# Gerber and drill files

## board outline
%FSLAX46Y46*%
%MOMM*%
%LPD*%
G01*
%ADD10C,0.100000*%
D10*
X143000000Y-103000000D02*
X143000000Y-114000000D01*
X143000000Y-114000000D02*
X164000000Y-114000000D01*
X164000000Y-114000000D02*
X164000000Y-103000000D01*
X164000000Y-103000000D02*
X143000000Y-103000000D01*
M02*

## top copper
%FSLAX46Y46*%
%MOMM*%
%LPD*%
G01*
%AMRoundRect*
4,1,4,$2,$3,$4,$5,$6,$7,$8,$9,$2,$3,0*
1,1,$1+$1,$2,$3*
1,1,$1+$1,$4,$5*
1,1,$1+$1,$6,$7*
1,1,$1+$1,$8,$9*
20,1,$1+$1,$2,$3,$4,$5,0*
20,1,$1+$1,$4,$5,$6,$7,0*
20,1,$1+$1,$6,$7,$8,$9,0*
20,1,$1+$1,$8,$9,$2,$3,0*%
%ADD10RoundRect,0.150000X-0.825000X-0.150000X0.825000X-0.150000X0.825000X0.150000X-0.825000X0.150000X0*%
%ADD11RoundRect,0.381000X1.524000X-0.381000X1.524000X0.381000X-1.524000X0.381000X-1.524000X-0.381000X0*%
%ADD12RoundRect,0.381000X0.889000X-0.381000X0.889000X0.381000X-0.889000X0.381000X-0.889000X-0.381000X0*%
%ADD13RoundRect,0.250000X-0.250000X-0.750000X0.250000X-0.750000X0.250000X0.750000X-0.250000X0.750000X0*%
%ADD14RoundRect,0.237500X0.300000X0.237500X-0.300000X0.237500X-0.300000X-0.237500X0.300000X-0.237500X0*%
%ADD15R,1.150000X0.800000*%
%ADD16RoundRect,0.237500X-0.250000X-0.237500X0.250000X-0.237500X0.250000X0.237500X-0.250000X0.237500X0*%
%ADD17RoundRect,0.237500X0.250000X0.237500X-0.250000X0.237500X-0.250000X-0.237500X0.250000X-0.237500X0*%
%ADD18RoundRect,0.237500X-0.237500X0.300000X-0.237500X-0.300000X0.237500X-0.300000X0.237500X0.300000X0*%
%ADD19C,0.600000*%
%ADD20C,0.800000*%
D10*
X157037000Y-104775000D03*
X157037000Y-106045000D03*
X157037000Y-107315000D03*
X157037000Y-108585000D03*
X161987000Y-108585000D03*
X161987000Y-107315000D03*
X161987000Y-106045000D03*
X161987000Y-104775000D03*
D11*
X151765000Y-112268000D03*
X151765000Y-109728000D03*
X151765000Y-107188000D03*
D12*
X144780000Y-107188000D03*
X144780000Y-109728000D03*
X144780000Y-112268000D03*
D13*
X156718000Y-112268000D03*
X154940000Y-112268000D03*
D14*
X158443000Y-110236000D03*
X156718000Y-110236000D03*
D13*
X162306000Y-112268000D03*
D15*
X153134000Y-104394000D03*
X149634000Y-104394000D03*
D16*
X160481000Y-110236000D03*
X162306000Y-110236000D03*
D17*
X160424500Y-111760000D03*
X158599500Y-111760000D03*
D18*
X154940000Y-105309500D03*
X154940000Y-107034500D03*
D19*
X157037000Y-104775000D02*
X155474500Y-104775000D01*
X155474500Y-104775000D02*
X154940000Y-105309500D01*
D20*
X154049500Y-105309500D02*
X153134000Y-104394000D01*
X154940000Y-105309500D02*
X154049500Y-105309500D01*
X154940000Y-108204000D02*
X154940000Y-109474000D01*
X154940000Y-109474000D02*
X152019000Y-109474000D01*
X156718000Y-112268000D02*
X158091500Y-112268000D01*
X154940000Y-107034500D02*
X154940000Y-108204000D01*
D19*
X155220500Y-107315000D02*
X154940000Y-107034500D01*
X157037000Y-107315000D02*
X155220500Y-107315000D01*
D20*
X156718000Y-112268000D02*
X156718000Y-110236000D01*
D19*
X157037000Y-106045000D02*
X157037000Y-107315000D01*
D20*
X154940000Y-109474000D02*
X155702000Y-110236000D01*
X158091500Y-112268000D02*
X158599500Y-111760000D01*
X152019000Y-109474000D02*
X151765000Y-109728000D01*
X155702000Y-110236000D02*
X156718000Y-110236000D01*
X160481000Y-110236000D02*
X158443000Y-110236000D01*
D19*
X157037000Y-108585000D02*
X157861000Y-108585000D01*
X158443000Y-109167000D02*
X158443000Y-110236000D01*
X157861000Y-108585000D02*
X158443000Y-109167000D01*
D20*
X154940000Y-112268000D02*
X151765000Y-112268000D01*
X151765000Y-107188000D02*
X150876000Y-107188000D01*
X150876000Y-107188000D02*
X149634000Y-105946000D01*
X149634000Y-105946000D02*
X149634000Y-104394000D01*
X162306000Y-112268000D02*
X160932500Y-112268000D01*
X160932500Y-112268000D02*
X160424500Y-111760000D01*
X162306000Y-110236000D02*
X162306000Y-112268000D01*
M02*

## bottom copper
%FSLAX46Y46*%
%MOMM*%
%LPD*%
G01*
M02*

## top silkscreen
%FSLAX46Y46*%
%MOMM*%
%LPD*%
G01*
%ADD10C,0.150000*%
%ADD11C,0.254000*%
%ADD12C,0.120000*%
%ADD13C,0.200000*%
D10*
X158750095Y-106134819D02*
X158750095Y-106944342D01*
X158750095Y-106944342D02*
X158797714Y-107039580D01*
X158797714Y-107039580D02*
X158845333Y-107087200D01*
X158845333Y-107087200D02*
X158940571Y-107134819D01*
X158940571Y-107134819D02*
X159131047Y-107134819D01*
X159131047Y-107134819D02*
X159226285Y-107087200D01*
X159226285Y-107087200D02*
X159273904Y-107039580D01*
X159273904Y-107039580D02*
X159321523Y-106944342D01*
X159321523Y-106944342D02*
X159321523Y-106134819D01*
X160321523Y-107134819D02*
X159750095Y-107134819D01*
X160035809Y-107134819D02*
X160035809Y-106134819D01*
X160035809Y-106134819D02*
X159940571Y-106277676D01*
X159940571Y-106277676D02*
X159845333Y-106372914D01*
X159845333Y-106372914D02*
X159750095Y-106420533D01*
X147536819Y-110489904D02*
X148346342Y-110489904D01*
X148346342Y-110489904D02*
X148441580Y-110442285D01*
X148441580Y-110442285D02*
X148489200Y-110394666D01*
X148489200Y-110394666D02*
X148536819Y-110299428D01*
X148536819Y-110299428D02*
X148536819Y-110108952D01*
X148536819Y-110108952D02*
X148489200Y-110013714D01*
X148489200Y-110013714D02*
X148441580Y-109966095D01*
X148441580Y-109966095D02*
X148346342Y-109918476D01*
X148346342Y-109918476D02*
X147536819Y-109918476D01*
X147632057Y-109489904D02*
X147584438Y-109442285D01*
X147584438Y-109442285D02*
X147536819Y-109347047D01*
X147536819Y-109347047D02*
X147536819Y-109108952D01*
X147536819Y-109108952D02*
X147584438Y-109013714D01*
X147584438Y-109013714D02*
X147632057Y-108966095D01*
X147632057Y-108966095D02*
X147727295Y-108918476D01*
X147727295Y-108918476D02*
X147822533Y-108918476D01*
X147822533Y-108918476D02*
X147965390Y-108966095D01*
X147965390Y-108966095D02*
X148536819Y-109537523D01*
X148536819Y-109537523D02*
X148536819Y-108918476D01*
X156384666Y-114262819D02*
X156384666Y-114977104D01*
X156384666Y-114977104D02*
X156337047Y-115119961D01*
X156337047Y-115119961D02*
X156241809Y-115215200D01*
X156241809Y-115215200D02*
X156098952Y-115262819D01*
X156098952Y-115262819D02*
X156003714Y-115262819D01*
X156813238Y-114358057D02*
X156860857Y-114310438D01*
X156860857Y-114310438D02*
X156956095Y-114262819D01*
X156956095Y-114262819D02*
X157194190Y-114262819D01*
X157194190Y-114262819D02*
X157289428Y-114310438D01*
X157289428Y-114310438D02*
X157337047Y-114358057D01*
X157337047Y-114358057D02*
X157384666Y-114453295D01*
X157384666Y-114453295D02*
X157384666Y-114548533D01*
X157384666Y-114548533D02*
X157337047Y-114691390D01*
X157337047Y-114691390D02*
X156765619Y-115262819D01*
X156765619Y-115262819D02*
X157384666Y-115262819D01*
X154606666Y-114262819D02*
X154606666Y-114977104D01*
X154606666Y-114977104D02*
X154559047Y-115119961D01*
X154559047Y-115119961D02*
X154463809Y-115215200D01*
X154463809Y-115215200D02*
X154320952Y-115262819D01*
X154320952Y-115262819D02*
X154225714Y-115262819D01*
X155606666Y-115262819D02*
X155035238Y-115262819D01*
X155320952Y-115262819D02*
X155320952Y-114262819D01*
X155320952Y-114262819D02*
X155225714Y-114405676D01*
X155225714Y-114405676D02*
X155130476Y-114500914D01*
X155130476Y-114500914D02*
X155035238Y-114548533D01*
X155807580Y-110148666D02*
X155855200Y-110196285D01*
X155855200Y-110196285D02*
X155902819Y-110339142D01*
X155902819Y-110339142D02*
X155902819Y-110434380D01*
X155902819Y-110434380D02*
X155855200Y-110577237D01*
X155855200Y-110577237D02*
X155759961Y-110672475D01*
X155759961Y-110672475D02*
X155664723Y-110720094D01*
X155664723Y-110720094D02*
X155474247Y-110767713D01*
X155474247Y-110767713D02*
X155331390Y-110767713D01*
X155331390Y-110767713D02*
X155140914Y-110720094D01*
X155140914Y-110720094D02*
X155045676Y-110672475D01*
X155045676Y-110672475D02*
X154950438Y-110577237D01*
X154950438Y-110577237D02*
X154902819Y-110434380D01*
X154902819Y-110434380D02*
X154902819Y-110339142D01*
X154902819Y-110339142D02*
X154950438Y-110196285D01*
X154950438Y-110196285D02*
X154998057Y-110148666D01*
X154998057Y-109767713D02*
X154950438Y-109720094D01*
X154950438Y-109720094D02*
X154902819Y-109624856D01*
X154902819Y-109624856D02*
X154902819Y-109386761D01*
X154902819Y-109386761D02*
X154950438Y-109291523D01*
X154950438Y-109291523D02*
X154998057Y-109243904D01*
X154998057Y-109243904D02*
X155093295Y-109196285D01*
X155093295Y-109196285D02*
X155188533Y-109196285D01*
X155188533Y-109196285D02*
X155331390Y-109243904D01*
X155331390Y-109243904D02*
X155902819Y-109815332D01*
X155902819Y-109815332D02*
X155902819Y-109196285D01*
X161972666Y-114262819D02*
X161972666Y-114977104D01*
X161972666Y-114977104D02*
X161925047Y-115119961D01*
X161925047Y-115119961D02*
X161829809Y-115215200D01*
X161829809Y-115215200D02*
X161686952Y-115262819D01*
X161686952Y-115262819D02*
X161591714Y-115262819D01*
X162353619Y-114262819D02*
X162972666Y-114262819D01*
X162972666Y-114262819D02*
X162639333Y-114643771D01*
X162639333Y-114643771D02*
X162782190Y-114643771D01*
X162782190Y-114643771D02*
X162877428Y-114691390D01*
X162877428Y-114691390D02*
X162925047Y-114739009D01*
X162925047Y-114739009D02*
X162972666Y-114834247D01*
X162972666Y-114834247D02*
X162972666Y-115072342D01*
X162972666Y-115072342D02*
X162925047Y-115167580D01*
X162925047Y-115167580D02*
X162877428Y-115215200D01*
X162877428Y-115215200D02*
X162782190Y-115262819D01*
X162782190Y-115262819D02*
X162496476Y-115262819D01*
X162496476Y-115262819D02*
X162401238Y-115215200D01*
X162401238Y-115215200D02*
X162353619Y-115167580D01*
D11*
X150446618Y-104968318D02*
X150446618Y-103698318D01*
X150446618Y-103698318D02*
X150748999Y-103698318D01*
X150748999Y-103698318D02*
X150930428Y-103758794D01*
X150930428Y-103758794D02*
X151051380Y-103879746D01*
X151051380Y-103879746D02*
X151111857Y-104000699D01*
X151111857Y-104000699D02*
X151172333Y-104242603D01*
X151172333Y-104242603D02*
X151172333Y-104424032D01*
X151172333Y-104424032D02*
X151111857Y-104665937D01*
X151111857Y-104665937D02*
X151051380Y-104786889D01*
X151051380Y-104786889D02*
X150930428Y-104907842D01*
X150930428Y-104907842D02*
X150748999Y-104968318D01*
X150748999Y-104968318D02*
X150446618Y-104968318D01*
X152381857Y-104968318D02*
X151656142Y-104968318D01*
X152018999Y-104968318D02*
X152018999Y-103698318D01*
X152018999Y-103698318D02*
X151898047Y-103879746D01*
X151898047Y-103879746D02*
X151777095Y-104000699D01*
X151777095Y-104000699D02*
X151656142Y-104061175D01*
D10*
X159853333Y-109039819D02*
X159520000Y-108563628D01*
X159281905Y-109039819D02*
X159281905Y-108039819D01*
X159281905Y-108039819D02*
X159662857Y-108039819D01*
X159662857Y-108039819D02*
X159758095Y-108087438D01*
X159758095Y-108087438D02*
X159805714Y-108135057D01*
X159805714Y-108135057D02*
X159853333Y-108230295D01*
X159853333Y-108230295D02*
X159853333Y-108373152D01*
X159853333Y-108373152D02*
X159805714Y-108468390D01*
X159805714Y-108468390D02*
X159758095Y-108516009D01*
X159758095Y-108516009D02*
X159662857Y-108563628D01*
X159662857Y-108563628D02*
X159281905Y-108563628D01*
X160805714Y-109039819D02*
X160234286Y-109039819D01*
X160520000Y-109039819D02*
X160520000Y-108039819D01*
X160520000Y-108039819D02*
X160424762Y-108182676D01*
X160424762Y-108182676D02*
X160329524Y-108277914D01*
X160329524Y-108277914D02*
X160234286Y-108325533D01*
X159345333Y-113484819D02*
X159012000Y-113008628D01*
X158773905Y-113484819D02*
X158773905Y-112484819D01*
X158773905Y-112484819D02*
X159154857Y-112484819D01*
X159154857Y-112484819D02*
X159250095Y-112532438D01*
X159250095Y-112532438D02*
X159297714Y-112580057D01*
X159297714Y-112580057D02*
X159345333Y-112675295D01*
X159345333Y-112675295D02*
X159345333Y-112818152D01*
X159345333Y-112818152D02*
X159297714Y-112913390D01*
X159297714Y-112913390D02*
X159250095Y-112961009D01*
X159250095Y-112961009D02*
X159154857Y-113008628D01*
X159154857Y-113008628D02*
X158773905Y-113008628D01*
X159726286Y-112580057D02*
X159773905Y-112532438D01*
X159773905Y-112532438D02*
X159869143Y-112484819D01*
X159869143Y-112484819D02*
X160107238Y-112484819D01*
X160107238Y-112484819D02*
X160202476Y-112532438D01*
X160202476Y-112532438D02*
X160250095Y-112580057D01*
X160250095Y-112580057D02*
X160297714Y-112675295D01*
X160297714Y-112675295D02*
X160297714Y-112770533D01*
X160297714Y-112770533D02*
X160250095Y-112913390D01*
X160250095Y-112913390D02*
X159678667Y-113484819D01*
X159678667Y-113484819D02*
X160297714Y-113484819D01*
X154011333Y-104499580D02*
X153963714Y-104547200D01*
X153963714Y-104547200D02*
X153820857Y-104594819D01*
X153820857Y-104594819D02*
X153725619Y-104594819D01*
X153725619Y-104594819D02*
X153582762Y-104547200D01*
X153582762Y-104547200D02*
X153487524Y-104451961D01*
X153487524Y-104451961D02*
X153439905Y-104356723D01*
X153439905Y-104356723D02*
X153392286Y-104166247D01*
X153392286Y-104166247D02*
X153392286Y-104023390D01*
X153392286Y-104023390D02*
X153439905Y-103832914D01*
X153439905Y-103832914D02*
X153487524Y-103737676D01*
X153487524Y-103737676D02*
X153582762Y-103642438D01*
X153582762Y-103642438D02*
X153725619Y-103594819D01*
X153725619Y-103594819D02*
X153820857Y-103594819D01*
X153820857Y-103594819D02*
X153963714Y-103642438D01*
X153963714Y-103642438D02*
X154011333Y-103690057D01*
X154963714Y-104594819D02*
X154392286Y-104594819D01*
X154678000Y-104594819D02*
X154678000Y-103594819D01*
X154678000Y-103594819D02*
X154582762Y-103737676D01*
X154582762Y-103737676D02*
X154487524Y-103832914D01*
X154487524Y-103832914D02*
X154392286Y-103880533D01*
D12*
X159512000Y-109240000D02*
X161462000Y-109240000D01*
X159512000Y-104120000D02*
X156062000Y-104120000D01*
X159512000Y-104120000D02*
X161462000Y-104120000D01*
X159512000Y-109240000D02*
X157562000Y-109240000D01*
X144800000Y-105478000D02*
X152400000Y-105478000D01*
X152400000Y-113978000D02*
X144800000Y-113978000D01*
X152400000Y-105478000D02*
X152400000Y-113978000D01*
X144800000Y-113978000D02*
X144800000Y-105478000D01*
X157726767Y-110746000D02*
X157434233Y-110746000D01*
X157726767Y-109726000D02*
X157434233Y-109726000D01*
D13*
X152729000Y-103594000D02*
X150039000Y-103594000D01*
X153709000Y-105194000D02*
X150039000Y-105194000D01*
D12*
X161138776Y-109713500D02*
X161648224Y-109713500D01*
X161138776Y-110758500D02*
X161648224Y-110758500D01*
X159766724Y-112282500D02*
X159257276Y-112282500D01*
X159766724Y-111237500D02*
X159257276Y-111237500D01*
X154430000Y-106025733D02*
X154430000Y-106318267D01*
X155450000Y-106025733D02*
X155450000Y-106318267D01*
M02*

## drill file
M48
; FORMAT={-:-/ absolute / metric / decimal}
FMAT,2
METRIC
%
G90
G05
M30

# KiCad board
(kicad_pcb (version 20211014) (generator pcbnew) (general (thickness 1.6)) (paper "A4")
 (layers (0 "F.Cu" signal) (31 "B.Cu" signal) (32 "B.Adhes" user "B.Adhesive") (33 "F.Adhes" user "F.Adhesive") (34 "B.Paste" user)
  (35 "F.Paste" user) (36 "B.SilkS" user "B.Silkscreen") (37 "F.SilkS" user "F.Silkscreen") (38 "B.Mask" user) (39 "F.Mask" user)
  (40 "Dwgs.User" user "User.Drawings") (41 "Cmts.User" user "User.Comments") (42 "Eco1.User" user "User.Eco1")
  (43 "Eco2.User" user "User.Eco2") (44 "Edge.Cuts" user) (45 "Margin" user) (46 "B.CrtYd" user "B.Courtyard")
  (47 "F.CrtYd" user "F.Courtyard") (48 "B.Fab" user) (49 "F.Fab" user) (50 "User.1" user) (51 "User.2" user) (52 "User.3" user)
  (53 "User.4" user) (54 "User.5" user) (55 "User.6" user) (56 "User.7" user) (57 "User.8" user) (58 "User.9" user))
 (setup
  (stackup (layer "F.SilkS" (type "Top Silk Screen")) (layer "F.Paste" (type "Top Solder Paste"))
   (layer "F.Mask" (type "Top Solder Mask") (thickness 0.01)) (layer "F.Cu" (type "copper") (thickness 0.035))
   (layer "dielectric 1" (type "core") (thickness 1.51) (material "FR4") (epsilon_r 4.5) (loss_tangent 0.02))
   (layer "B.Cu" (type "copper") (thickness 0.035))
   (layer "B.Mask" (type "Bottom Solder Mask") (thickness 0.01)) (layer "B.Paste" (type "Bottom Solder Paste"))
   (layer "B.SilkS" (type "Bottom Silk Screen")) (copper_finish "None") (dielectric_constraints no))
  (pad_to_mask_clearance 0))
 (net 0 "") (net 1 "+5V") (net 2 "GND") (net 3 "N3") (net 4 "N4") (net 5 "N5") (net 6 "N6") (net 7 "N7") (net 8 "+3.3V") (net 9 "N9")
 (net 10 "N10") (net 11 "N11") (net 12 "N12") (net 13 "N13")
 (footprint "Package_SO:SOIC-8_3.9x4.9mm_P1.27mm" (layer "F.Cu") (at 159.512 106.68)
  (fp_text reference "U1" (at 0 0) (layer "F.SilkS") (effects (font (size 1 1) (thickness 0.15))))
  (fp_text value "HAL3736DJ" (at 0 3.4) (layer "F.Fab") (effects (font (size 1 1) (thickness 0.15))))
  (fp_line (start 0 2.56) (end 1.95 2.56) (layer "F.SilkS") (width 0.12))
  (fp_line (start 0 -2.56) (end -3.45 -2.56) (layer "F.SilkS") (width 0.12))
  (fp_line (start 0 -2.56) (end 1.95 -2.56) (layer "F.SilkS") (width 0.12))
  (fp_line (start 0 2.56) (end -1.95 2.56) (layer "F.SilkS") (width 0.12))
  (pad "1" smd roundrect (at -2.475 -1.905) (size 1.95 0.6) (layers "F.Cu" "F.Paste" "F.Mask") (roundrect_rratio 0.25) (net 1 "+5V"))
  (pad "2" smd roundrect (at -2.475 -0.635) (size 1.95 0.6) (layers "F.Cu" "F.Paste" "F.Mask") (roundrect_rratio 0.25) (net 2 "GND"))
  (pad "3" smd roundrect (at -2.475 0.635) (size 1.95 0.6) (layers "F.Cu" "F.Paste" "F.Mask") (roundrect_rratio 0.25) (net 2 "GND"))
  (pad "4" smd roundrect (at -2.475 1.905) (size 1.95 0.6) (layers "F.Cu" "F.Paste" "F.Mask") (roundrect_rratio 0.25) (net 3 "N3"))
  (pad "5" smd roundrect (at 2.475 1.905) (size 1.95 0.6) (layers "F.Cu" "F.Paste" "F.Mask") (roundrect_rratio 0.25) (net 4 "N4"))
  (pad "6" smd roundrect (at 2.475 0.635) (size 1.95 0.6) (layers "F.Cu" "F.Paste" "F.Mask") (roundrect_rratio 0.25) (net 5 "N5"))
  (pad "7" smd roundrect (at 2.475 -0.635) (size 1.95 0.6) (layers "F.Cu" "F.Paste" "F.Mask") (roundrect_rratio 0.25) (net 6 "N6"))
  (pad "8" smd roundrect (at 2.475 -1.905) (size 1.95 0.6) (layers "F.Cu" "F.Paste" "F.Mask") (roundrect_rratio 0.25) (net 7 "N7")))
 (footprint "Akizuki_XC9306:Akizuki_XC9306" (layer "F.Cu") (at 144.8 109.728 90)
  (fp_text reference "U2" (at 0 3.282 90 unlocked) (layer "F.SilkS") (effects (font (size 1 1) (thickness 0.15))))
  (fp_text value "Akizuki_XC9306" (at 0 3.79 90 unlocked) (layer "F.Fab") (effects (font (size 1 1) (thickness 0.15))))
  (fp_line (start 4.25 0) (end 4.25 7.6) (layer "F.SilkS") (width 0.12))
  (fp_line (start -4.25 7.6) (end -4.25 0) (layer "F.SilkS") (width 0.12))
  (fp_line (start 4.25 7.6) (end -4.25 7.6) (layer "F.SilkS") (width 0.12))
  (fp_line (start -4.25 0) (end 4.25 0) (layer "F.SilkS") (width 0.12))
  (pad "1" smd roundrect (at -2.54 6.965 90) (size 1.524 3.81) (layers "F.Cu" "F.Paste" "F.Mask") (roundrect_rratio 0.25) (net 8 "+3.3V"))
  (pad "2" smd roundrect (at 0 6.965 90) (size 1.524 3.81) (layers "F.Cu" "F.Paste" "F.Mask") (roundrect_rratio 0.25) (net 2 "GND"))
  (pad "3" smd roundrect (at 2.54 6.965 90) (size 1.524 3.81) (layers "F.Cu" "F.Paste" "F.Mask") (roundrect_rratio 0.25) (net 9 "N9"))
  (pad "4" smd roundrect (at 2.54 -0.02 90) (size 1.524 2.54) (layers "F.Cu" "F.Paste" "F.Mask") (roundrect_rratio 0.25) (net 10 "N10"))
  (pad "5" smd roundrect (at 0 -0.02 90) (size 1.524 2.54) (layers "F.Cu" "F.Paste" "F.Mask") (roundrect_rratio 0.25) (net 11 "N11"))
  (pad "6" smd roundrect (at -2.54 -0.02 90) (size 1.524 2.54) (layers "F.Cu" "F.Paste" "F.Mask") (roundrect_rratio 0.25) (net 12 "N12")))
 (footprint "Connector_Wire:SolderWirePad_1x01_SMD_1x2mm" (layer "F.Cu") (at 156.718 112.268)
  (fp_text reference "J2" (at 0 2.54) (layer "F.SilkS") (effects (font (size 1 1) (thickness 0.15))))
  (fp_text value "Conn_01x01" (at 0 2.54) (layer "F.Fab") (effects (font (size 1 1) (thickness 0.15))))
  (pad "1" smd roundrect (at 0 0) (size 1 2) (layers "F.Cu" "F.Paste" "F.Mask") (roundrect_rratio 0.25) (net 2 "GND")))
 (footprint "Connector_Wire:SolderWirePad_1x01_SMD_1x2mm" (layer "F.Cu") (at 154.94 112.268)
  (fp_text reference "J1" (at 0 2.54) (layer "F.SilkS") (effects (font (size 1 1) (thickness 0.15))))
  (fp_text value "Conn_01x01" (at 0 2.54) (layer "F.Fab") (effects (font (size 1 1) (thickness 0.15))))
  (pad "1" smd roundrect (at 0 0) (size 1 2) (layers "F.Cu" "F.Paste" "F.Mask") (roundrect_rratio 0.25) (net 8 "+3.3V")))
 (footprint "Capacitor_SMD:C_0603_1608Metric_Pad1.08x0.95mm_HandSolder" (layer "F.Cu") (at 157.5805 110.236 180)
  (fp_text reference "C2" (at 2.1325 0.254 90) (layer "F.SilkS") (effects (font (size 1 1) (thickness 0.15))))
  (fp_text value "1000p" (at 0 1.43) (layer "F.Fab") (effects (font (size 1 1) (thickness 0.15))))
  (fp_line (start -0.146267 -0.51) (end 0.146267 -0.51) (layer "F.SilkS") (width 0.12))
  (fp_line (start -0.146267 0.51) (end 0.146267 0.51) (layer "F.SilkS") (width 0.12))
  (pad "1" smd roundrect (at -0.8625 0 180) (size 1.075 0.95) (layers "F.Cu" "F.Paste" "F.Mask") (roundrect_rratio 0.25) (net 3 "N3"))
  (pad "2" smd roundrect (at 0.8625 0 180) (size 1.075 0.95) (layers "F.Cu" "F.Paste" "F.Mask") (roundrect_rratio 0.25) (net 2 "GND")))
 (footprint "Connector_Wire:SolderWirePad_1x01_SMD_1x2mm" (layer "F.Cu") (at 162.306 112.268)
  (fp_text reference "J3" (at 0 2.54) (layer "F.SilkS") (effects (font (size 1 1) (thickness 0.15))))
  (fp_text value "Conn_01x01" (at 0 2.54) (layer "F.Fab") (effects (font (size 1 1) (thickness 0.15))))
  (pad "1" smd roundrect (at 0 0) (size 1 2) (layers "F.Cu" "F.Paste" "F.Mask") (roundrect_rratio 0.25) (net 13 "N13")))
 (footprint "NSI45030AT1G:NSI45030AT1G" (layer "F.Cu") (at 151.384 104.394 180)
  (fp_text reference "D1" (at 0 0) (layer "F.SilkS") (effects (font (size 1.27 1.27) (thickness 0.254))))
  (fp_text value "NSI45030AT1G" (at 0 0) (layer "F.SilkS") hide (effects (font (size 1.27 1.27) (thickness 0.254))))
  (fp_line (start -1.345 0.8) (end 1.345 0.8) (layer "F.SilkS") (width 0.2))
  (fp_line (start -2.325 -0.8) (end 1.345 -0.8) (layer "F.SilkS") (width 0.2))
  (pad "1" smd rect locked (at -1.75 0 270) (size 0.8 1.15) (layers "F.Cu" "F.Paste" "F.Mask") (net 1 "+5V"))
  (pad "2" smd rect locked (at 1.75 0 270) (size 0.8 1.15) (layers "F.Cu" "F.Paste" "F.Mask") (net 9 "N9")))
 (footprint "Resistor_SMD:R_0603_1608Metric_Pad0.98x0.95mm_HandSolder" (layer "F.Cu") (at 161.3935 110.236)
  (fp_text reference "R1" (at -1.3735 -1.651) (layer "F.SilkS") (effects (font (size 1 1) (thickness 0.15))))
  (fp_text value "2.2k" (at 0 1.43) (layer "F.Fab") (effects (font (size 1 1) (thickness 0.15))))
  (fp_line (start -0.254724 -0.5225) (end 0.254724 -0.5225) (layer "F.SilkS") (width 0.12))
  (fp_line (start -0.254724 0.5225) (end 0.254724 0.5225) (layer "F.SilkS") (width 0.12))
  (pad "1" smd roundrect (at -0.9125 0) (size 0.975 0.95) (layers "F.Cu" "F.Paste" "F.Mask") (roundrect_rratio 0.25) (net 3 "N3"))
  (pad "2" smd roundrect (at 0.9125 0) (size 0.975 0.95) (layers "F.Cu" "F.Paste" "F.Mask") (roundrect_rratio 0.25) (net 13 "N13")))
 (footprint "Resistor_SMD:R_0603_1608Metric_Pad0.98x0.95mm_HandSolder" (layer "F.Cu") (at 159.512 111.76 180)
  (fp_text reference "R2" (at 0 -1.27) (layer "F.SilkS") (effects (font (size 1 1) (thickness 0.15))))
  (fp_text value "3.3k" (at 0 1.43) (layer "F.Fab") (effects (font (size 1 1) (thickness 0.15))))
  (fp_line (start -0.254724 -0.5225) (end 0.254724 -0.5225) (layer "F.SilkS") (width 0.12))
  (fp_line (start -0.254724 0.5225) (end 0.254724 0.5225) (layer "F.SilkS") (width 0.12))
  (pad "1" smd roundrect (at -0.9125 0 180) (size 0.975 0.95) (layers "F.Cu" "F.Paste" "F.Mask") (roundrect_rratio 0.25) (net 13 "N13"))
  (pad "2" smd roundrect (at 0.9125 0 180) (size 0.975 0.95) (layers "F.Cu" "F.Paste" "F.Mask") (roundrect_rratio 0.25) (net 2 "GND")))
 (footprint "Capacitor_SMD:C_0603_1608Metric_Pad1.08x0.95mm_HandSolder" (layer "F.Cu") (at 154.94 106.172 -90)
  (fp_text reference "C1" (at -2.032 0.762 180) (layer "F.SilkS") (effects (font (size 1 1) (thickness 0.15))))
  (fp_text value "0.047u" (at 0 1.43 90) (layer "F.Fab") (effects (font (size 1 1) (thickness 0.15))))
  (fp_line (start -0.146267 0.51) (end 0.146267 0.51) (layer "F.SilkS") (width 0.12))
  (fp_line (start -0.146267 -0.51) (end 0.146267 -0.51) (layer "F.SilkS") (width 0.12))
  (pad "1" smd roundrect (at -0.8625 0 270) (size 1.075 0.95) (layers "F.Cu" "F.Paste" "F.Mask") (roundrect_rratio 0.25) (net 1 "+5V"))
  (pad "2" smd roundrect (at 0.8625 0 270) (size 1.075 0.95) (layers "F.Cu" "F.Paste" "F.Mask") (roundrect_rratio 0.25) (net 2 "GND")))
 (gr_line (start 143 103) (end 143 114) (layer "Edge.Cuts") (width 0.1))
 (gr_line (start 143 114) (end 164 114) (layer "Edge.Cuts") (width 0.1))
 (gr_line (start 164 114) (end 164 103) (layer "Edge.Cuts") (width 0.1))
 (gr_line (start 164 103) (end 143 103) (layer "Edge.Cuts") (width 0.1))
 (segment (start 157.037 104.775) (end 155.4745 104.775) (width 0.6) (layer "F.Cu") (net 1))
 (segment (start 155.4745 104.775) (end 154.94 105.3095) (width 0.6) (layer "F.Cu") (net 1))
 (segment (start 154.0495 105.3095) (end 153.134 104.394) (width 0.8) (layer "F.Cu") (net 1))
 (segment (start 154.94 105.3095) (end 154.0495 105.3095) (width 0.8) (layer "F.Cu") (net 1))
 (segment (start 154.94 108.204) (end 154.94 109.474) (width 0.8) (layer "F.Cu") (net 2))
 (segment (start 154.94 109.474) (end 152.019 109.474) (width 0.8) (layer "F.Cu") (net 2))
 (segment (start 156.718 112.268) (end 158.0915 112.268) (width 0.8) (layer "F.Cu") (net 2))
 (segment (start 154.94 107.0345) (end 154.94 108.204) (width 0.8) (layer "F.Cu") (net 2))
 (segment (start 155.2205 107.315) (end 154.94 107.0345) (width 0.6) (layer "F.Cu") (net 2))
 (segment (start 157.037 107.315) (end 155.2205 107.315) (width 0.6) (layer "F.Cu") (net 2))
 (segment (start 156.718 112.268) (end 156.718 110.236) (width 0.8) (layer "F.Cu") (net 2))
 (segment (start 157.037 106.045) (end 157.037 107.315) (width 0.6) (layer "F.Cu") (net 2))
 (segment (start 154.94 109.474) (end 155.702 110.236) (width 0.8) (layer "F.Cu") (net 2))
 (segment (start 158.0915 112.268) (end 158.5995 111.76) (width 0.8) (layer "F.Cu") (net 2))
 (segment (start 152.019 109.474) (end 151.765 109.728) (width 0.8) (layer "F.Cu") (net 2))
 (segment (start 155.702 110.236) (end 156.718 110.236) (width 0.8) (layer "F.Cu") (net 2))
 (segment (start 160.481 110.236) (end 158.443 110.236) (width 0.8) (layer "F.Cu") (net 3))
 (segment (start 157.037 108.585) (end 157.861 108.585) (width 0.6) (layer "F.Cu") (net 3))
 (segment (start 158.443 109.167) (end 158.443 110.236) (width 0.6) (layer "F.Cu") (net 3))
 (segment (start 157.861 108.585) (end 158.443 109.167) (width 0.6) (layer "F.Cu") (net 3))
 (segment (start 154.94 112.268) (end 151.765 112.268) (width 0.8) (layer "F.Cu") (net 8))
 (segment (start 151.765 107.188) (end 150.876 107.188) (width 0.8) (layer "F.Cu") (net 9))
 (segment (start 150.876 107.188) (end 149.634 105.946) (width 0.8) (layer "F.Cu") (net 9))
 (segment (start 149.634 105.946) (end 149.634 104.394) (width 0.8) (layer "F.Cu") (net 9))
 (segment (start 162.306 112.268) (end 160.9325 112.268) (width 0.8) (layer "F.Cu") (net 13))
 (segment (start 160.9325 112.268) (end 160.4245 111.76) (width 0.8) (layer "F.Cu") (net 13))
 (segment (start 162.306 110.236) (end 162.306 112.268) (width 0.8) (layer "F.Cu") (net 13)))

